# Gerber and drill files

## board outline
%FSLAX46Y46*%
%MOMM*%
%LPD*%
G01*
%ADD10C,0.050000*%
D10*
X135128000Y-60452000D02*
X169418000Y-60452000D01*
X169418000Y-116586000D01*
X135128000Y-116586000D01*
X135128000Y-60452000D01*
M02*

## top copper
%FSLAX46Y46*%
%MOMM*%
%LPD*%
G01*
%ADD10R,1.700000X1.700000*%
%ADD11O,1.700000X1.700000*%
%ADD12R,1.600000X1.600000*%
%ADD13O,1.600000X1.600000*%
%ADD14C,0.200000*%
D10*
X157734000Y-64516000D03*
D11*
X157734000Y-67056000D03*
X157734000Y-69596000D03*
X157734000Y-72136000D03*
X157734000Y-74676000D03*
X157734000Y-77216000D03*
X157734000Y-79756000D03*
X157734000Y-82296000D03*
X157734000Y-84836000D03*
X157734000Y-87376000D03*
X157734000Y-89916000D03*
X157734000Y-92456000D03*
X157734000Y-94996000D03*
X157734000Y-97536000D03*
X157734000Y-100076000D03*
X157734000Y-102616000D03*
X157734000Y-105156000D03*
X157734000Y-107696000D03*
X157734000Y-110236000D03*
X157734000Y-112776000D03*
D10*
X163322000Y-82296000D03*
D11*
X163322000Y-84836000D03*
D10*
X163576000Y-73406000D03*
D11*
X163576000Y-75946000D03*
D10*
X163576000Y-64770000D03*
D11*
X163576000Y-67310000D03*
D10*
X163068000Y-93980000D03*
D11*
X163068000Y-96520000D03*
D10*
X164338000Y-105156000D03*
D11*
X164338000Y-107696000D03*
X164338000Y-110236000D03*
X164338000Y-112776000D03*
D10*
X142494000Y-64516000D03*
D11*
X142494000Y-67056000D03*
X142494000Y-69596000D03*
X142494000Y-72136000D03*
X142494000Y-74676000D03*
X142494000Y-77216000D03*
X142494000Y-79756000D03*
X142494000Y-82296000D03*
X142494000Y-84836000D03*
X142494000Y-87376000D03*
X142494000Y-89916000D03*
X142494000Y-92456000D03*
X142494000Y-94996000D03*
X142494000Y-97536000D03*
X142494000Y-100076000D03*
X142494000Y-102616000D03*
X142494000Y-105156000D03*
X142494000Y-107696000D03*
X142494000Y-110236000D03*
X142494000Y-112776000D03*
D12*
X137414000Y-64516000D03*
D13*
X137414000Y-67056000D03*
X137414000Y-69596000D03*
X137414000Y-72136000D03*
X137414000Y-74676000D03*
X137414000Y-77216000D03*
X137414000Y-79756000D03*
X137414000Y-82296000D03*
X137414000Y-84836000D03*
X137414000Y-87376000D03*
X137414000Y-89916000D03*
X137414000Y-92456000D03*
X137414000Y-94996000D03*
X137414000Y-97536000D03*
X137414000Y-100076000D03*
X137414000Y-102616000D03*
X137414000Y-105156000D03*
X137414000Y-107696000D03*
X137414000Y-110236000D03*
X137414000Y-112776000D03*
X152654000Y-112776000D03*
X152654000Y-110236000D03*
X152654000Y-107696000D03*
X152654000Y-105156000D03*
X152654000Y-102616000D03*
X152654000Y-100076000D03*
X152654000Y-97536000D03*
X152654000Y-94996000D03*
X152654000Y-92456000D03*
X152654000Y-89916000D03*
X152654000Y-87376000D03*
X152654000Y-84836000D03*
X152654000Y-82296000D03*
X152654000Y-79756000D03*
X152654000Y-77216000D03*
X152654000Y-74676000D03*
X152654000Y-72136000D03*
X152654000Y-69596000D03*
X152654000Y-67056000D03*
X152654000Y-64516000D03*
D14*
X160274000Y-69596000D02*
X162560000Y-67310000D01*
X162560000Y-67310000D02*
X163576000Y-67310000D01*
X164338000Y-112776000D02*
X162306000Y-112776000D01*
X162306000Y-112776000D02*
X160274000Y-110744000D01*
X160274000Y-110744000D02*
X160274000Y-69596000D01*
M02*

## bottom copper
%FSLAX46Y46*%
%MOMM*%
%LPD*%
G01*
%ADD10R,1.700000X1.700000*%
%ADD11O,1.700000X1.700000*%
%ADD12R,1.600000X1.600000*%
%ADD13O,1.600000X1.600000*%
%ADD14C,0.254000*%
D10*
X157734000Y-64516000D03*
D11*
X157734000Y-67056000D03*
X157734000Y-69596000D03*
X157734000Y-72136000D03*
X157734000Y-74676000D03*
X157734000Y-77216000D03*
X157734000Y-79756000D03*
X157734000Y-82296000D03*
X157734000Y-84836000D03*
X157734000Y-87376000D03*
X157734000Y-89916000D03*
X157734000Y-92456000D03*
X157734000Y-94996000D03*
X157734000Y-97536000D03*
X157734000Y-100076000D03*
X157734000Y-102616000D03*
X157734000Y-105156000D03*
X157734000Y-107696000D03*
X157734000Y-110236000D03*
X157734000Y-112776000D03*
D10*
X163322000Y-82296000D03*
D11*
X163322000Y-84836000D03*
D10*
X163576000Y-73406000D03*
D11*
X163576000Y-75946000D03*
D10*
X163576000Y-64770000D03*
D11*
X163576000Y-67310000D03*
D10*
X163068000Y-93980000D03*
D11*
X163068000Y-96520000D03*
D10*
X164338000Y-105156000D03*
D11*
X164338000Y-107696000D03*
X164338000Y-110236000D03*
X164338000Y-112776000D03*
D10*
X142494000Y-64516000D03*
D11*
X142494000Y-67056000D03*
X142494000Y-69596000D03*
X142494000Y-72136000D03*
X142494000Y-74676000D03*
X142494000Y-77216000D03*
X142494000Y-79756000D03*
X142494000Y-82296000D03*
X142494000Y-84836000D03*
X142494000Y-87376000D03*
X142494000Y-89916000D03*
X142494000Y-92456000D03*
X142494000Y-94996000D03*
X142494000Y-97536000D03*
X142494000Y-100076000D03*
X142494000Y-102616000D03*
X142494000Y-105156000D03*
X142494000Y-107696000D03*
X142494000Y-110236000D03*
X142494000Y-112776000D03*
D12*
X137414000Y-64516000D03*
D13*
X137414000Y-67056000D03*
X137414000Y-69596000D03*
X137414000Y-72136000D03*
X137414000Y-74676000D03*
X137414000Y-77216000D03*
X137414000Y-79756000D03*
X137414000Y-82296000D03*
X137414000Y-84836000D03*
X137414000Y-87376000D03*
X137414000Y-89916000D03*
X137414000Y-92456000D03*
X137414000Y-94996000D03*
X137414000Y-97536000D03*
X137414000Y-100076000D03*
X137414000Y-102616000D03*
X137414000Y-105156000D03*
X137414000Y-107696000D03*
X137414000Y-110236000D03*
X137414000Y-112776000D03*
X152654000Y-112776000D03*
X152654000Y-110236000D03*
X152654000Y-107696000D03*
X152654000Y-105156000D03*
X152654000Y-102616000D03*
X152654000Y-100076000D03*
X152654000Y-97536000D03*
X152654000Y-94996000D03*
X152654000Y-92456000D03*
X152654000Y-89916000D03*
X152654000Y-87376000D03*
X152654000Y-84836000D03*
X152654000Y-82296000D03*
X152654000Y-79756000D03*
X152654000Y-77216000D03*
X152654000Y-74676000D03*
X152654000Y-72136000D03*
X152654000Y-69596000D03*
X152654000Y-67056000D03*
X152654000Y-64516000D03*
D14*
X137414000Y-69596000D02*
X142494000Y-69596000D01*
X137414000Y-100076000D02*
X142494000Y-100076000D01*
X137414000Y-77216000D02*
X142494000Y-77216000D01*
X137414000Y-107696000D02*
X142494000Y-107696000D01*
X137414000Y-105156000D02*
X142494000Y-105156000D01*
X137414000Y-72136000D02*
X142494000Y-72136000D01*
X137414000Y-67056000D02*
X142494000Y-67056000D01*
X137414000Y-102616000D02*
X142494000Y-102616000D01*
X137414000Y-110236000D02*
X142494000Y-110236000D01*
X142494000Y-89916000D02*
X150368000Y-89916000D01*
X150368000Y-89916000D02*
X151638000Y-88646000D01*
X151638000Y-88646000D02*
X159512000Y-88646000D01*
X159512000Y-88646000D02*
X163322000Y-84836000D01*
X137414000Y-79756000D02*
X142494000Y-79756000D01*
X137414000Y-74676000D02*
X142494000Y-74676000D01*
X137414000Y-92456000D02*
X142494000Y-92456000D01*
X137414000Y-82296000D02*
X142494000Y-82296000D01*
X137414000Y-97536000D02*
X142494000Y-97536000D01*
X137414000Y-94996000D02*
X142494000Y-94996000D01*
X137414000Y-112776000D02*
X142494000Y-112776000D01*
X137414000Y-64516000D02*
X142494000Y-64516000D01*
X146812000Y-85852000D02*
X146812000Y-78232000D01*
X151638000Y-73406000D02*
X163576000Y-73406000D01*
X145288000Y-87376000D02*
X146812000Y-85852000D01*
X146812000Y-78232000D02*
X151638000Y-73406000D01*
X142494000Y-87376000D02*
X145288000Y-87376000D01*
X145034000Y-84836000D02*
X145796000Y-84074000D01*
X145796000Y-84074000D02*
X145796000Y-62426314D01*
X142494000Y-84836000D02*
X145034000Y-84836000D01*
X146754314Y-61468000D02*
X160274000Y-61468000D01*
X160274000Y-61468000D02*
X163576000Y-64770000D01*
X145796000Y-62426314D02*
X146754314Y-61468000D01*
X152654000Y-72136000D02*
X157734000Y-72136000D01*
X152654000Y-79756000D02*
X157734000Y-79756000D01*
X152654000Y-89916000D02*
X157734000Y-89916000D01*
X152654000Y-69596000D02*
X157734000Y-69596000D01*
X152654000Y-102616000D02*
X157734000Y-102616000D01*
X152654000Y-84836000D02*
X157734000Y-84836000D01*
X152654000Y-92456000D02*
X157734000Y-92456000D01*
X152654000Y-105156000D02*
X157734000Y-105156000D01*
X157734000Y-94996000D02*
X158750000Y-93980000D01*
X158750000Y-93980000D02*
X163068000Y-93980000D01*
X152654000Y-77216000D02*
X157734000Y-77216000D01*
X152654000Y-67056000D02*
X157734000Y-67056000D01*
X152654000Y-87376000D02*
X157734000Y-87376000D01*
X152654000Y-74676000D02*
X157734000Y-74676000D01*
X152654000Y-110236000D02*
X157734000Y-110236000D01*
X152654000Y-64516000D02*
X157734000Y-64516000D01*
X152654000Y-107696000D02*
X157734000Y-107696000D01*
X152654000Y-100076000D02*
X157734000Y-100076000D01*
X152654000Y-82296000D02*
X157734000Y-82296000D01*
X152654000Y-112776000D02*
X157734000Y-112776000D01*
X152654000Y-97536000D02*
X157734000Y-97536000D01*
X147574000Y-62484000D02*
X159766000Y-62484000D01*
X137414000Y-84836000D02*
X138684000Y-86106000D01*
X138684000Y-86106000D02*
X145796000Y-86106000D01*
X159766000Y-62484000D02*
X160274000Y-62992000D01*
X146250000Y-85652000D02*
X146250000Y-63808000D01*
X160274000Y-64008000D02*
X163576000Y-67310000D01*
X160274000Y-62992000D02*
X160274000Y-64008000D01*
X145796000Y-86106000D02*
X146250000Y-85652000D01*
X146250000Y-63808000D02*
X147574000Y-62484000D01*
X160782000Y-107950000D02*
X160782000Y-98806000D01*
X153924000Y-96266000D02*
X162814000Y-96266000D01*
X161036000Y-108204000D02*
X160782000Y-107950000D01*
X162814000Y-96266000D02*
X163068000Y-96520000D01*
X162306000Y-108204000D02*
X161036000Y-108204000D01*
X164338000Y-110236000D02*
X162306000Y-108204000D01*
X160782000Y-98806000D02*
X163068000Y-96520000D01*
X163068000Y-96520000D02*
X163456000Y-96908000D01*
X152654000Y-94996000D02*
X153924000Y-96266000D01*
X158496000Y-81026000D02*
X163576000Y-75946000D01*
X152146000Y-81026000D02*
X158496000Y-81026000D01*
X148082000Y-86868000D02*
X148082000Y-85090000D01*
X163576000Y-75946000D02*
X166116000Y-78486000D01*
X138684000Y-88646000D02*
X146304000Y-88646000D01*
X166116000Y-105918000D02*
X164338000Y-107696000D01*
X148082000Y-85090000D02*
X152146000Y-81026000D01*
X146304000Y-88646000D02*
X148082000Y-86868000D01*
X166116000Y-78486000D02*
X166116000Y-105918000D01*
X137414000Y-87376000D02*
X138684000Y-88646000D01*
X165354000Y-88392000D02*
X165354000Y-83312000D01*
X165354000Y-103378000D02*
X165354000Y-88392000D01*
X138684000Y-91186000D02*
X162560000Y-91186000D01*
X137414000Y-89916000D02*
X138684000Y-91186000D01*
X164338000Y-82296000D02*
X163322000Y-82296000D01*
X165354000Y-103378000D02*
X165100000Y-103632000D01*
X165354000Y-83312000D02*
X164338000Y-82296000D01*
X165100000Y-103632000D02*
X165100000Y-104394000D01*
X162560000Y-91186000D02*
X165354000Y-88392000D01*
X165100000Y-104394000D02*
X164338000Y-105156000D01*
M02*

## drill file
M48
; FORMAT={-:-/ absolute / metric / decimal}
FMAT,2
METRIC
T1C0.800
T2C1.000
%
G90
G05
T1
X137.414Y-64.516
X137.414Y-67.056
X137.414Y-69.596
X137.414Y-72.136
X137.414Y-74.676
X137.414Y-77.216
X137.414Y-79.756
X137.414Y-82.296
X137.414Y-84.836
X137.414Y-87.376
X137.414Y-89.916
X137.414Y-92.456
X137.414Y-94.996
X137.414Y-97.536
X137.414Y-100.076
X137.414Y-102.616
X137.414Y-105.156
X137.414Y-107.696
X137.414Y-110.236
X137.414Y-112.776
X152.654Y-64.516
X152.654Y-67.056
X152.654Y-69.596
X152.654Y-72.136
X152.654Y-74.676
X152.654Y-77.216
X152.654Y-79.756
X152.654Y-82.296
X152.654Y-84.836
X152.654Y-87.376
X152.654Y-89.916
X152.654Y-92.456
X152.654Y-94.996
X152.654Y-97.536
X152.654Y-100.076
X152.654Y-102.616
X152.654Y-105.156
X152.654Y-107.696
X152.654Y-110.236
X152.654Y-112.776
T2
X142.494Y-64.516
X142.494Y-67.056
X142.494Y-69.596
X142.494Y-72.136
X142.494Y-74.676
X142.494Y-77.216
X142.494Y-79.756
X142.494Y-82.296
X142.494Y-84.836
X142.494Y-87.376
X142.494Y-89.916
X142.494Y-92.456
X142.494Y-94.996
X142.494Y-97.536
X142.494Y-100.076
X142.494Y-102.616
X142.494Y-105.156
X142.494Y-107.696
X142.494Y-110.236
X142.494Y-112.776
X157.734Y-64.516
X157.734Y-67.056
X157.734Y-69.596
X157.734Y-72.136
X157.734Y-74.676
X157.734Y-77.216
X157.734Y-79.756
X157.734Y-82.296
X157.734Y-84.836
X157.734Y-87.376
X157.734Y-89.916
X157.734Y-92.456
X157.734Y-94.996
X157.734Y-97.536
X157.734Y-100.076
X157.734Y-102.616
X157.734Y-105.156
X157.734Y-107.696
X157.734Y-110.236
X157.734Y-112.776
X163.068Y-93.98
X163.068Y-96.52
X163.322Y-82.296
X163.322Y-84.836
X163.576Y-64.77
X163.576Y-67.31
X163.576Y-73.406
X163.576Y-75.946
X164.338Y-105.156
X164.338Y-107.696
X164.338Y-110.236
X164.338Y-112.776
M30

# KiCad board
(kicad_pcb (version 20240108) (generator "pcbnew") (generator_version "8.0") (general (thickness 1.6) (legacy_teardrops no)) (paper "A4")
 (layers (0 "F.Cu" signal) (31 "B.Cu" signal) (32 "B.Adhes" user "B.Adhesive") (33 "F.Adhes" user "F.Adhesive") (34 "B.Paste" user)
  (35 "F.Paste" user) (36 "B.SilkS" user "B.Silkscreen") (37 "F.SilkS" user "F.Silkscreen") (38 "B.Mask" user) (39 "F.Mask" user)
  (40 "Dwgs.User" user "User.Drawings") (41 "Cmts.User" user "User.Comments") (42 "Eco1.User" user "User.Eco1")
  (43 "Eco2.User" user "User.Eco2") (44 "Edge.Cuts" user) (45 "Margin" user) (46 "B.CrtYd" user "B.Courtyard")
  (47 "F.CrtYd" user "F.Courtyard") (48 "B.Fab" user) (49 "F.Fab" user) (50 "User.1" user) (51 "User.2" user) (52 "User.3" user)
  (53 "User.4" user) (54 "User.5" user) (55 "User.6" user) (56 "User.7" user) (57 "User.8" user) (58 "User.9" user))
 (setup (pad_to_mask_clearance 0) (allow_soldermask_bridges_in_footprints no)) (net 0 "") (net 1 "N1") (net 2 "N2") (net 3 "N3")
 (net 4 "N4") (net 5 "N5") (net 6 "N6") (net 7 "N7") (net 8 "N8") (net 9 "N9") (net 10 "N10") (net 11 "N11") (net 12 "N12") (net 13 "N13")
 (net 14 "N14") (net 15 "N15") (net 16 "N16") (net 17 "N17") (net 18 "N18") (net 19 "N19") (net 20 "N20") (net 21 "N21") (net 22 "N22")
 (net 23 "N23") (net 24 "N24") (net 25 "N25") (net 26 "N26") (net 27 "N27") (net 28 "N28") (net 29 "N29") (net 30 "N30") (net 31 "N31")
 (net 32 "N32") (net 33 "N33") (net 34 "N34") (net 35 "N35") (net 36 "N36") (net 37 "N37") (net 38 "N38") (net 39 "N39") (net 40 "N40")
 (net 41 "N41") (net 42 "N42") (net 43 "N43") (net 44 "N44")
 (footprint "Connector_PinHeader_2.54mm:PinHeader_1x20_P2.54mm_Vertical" (layer "F.Cu") (at 157.734 64.516)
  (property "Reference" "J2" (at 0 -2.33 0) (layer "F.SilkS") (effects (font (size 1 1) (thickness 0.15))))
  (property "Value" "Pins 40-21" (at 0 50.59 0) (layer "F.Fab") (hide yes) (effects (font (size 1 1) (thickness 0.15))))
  (pad "1" thru_hole rect (at 0 0) (size 1.7 1.7) (drill 1) (layers "*.Cu" "*.Mask") (remove_unused_layers no) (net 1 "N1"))
  (pad "2" thru_hole oval (at 0 2.54) (size 1.7 1.7) (drill 1) (layers "*.Cu" "*.Mask") (remove_unused_layers no) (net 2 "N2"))
  (pad "3" thru_hole oval (at 0 5.08) (size 1.7 1.7) (drill 1) (layers "*.Cu" "*.Mask") (remove_unused_layers no) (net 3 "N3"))
  (pad "4" thru_hole oval (at 0 7.62) (size 1.7 1.7) (drill 1) (layers "*.Cu" "*.Mask") (remove_unused_layers no) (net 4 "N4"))
  (pad "5" thru_hole oval (at 0 10.16) (size 1.7 1.7) (drill 1) (layers "*.Cu" "*.Mask") (remove_unused_layers no) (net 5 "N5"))
  (pad "6" thru_hole oval (at 0 12.7) (size 1.7 1.7) (drill 1) (layers "*.Cu" "*.Mask") (remove_unused_layers no) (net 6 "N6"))
  (pad "7" thru_hole oval (at 0 15.24) (size 1.7 1.7) (drill 1) (layers "*.Cu" "*.Mask") (remove_unused_layers no) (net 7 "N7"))
  (pad "8" thru_hole oval (at 0 17.78) (size 1.7 1.7) (drill 1) (layers "*.Cu" "*.Mask") (remove_unused_layers no) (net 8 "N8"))
  (pad "9" thru_hole oval (at 0 20.32) (size 1.7 1.7) (drill 1) (layers "*.Cu" "*.Mask") (remove_unused_layers no) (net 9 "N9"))
  (pad "10" thru_hole oval (at 0 22.86) (size 1.7 1.7) (drill 1) (layers "*.Cu" "*.Mask") (remove_unused_layers no) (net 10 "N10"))
  (pad "11" thru_hole oval (at 0 25.4) (size 1.7 1.7) (drill 1) (layers "*.Cu" "*.Mask") (remove_unused_layers no) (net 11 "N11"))
  (pad "12" thru_hole oval (at 0 27.94) (size 1.7 1.7) (drill 1) (layers "*.Cu" "*.Mask") (remove_unused_layers no) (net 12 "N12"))
  (pad "13" thru_hole oval (at 0 30.48) (size 1.7 1.7) (drill 1) (layers "*.Cu" "*.Mask") (remove_unused_layers no) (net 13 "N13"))
  (pad "14" thru_hole oval (at 0 33.02) (size 1.7 1.7) (drill 1) (layers "*.Cu" "*.Mask") (remove_unused_layers no) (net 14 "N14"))
  (pad "15" thru_hole oval (at 0 35.56) (size 1.7 1.7) (drill 1) (layers "*.Cu" "*.Mask") (remove_unused_layers no) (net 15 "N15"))
  (pad "16" thru_hole oval (at 0 38.1) (size 1.7 1.7) (drill 1) (layers "*.Cu" "*.Mask") (remove_unused_layers no) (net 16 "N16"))
  (pad "17" thru_hole oval (at 0 40.64) (size 1.7 1.7) (drill 1) (layers "*.Cu" "*.Mask") (remove_unused_layers no) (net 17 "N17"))
  (pad "18" thru_hole oval (at 0 43.18) (size 1.7 1.7) (drill 1) (layers "*.Cu" "*.Mask") (remove_unused_layers no) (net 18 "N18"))
  (pad "19" thru_hole oval (at 0 45.72) (size 1.7 1.7) (drill 1) (layers "*.Cu" "*.Mask") (remove_unused_layers no) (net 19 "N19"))
  (pad "20" thru_hole oval (at 0 48.26) (size 1.7 1.7) (drill 1) (layers "*.Cu" "*.Mask") (remove_unused_layers no) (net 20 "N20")))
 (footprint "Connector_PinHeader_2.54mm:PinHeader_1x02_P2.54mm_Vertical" (layer "F.Cu") (at 163.322 82.296)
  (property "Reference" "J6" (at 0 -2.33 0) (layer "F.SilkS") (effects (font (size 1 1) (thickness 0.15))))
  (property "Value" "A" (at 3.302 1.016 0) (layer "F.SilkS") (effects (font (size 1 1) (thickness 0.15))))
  (pad "1" thru_hole rect (at 0 0) (size 1.7 1.7) (drill 1) (layers "*.Cu" "*.Mask") (remove_unused_layers no) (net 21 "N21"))
  (pad "2" thru_hole oval (at 0 2.54) (size 1.7 1.7) (drill 1) (layers "*.Cu" "*.Mask") (remove_unused_layers no) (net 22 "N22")))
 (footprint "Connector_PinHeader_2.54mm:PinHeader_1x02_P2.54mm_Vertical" (layer "F.Cu") (at 163.576 73.406)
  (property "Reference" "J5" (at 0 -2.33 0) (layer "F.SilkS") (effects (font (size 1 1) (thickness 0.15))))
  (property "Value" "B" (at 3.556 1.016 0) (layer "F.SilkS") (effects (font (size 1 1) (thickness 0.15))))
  (pad "1" thru_hole rect (at 0 0) (size 1.7 1.7) (drill 1) (layers "*.Cu" "*.Mask") (remove_unused_layers no) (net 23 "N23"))
  (pad "2" thru_hole oval (at 0 2.54) (size 1.7 1.7) (drill 1) (layers "*.Cu" "*.Mask") (remove_unused_layers no) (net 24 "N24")))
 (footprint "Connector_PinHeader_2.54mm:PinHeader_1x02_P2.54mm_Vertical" (layer "F.Cu") (at 163.576 64.77)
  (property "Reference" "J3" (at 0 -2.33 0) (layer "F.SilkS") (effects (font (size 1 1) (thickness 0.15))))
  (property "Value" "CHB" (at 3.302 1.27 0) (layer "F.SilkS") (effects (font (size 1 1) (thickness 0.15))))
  (pad "1" thru_hole rect (at 0 0) (size 1.7 1.7) (drill 1) (layers "*.Cu" "*.Mask") (remove_unused_layers no) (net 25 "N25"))
  (pad "2" thru_hole oval (at 0 2.54) (size 1.7 1.7) (drill 1) (layers "*.Cu" "*.Mask") (remove_unused_layers no) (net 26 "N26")))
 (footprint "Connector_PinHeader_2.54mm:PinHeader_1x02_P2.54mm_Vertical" (layer "F.Cu") (at 163.068 93.98)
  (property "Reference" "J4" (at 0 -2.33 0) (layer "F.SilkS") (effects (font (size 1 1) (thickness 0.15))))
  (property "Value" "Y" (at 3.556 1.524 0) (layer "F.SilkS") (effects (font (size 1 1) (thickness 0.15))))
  (pad "1" thru_hole rect (at 0 0) (size 1.7 1.7) (drill 1) (layers "*.Cu" "*.Mask") (remove_unused_layers no) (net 13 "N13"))
  (pad "2" thru_hole oval (at 0 2.54) (size 1.7 1.7) (drill 1) (layers "*.Cu" "*.Mask") (remove_unused_layers no) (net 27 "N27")))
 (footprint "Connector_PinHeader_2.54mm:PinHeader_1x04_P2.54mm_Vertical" (layer "F.Cu") (at 164.338 105.156)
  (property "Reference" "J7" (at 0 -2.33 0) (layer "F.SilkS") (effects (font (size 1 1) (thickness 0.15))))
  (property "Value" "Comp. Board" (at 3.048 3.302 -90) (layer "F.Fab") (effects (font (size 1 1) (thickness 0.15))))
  (pad "1" thru_hole rect (at 0 0) (size 1.7 1.7) (drill 1) (layers "*.Cu" "*.Mask") (remove_unused_layers no) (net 21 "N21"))
  (pad "2" thru_hole oval (at 0 2.54) (size 1.7 1.7) (drill 1) (layers "*.Cu" "*.Mask") (remove_unused_layers no) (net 24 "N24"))
  (pad "3" thru_hole oval (at 0 5.08) (size 1.7 1.7) (drill 1) (layers "*.Cu" "*.Mask") (remove_unused_layers no) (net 27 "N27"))
  (pad "4" thru_hole oval (at 0 7.62) (size 1.7 1.7) (drill 1) (layers "*.Cu" "*.Mask") (remove_unused_layers no) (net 26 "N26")))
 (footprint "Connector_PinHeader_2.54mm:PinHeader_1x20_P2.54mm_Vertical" (layer "F.Cu") (at 142.494 64.516)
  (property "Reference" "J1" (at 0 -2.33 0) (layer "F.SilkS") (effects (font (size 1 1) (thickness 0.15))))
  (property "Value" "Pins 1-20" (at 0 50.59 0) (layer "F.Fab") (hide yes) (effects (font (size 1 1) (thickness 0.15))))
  (pad "1" thru_hole rect (at 0 0) (size 1.7 1.7) (drill 1) (layers "*.Cu" "*.Mask") (remove_unused_layers no) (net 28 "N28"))
  (pad "2" thru_hole oval (at 0 2.54) (size 1.7 1.7) (drill 1) (layers "*.Cu" "*.Mask") (remove_unused_layers no) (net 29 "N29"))
  (pad "3" thru_hole oval (at 0 5.08) (size 1.7 1.7) (drill 1) (layers "*.Cu" "*.Mask") (remove_unused_layers no) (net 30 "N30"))
  (pad "4" thru_hole oval (at 0 7.62) (size 1.7 1.7) (drill 1) (layers "*.Cu" "*.Mask") (remove_unused_layers no) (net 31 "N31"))
  (pad "5" thru_hole oval (at 0 10.16) (size 1.7 1.7) (drill 1) (layers "*.Cu" "*.Mask") (remove_unused_layers no) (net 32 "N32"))
  (pad "6" thru_hole oval (at 0 12.7) (size 1.7 1.7) (drill 1) (layers "*.Cu" "*.Mask") (remove_unused_layers no) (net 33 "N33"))
  (pad "7" thru_hole oval (at 0 15.24) (size 1.7 1.7) (drill 1) (layers "*.Cu" "*.Mask") (remove_unused_layers no) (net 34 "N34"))
  (pad "8" thru_hole oval (at 0 17.78) (size 1.7 1.7) (drill 1) (layers "*.Cu" "*.Mask") (remove_unused_layers no) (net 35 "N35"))
  (pad "9" thru_hole oval (at 0 20.32) (size 1.7 1.7) (drill 1) (layers "*.Cu" "*.Mask") (remove_unused_layers no) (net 25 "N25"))
  (pad "10" thru_hole oval (at 0 22.86) (size 1.7 1.7) (drill 1) (layers "*.Cu" "*.Mask") (remove_unused_layers no) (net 23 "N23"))
  (pad "11" thru_hole oval (at 0 25.4) (size 1.7 1.7) (drill 1) (layers "*.Cu" "*.Mask") (remove_unused_layers no) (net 22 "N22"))
  (pad "12" thru_hole oval (at 0 27.94) (size 1.7 1.7) (drill 1) (layers "*.Cu" "*.Mask") (remove_unused_layers no) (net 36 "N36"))
  (pad "13" thru_hole oval (at 0 30.48) (size 1.7 1.7) (drill 1) (layers "*.Cu" "*.Mask") (remove_unused_layers no) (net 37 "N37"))
  (pad "14" thru_hole oval (at 0 33.02) (size 1.7 1.7) (drill 1) (layers "*.Cu" "*.Mask") (remove_unused_layers no) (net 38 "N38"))
  (pad "15" thru_hole oval (at 0 35.56) (size 1.7 1.7) (drill 1) (layers "*.Cu" "*.Mask") (remove_unused_layers no) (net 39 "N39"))
  (pad "16" thru_hole oval (at 0 38.1) (size 1.7 1.7) (drill 1) (layers "*.Cu" "*.Mask") (remove_unused_layers no) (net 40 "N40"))
  (pad "17" thru_hole oval (at 0 40.64) (size 1.7 1.7) (drill 1) (layers "*.Cu" "*.Mask") (remove_unused_layers no) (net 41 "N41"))
  (pad "18" thru_hole oval (at 0 43.18) (size 1.7 1.7) (drill 1) (layers "*.Cu" "*.Mask") (remove_unused_layers no) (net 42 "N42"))
  (pad "19" thru_hole oval (at 0 45.72) (size 1.7 1.7) (drill 1) (layers "*.Cu" "*.Mask") (remove_unused_layers no) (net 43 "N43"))
  (pad "20" thru_hole oval (at 0 48.26) (size 1.7 1.7) (drill 1) (layers "*.Cu" "*.Mask") (remove_unused_layers no) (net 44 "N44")))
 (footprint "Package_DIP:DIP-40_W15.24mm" (layer "F.Cu") (at 137.414 64.516)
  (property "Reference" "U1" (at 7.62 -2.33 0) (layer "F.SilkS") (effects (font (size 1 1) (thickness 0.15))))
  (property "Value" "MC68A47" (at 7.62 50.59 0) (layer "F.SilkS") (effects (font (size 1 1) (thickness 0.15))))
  (pad "1" thru_hole rect (at 0 0) (size 1.6 1.6) (drill 0.8) (layers "*.Cu" "*.Mask") (remove_unused_layers no) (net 28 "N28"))
  (pad "2" thru_hole oval (at 0 2.54) (size 1.6 1.6) (drill 0.8) (layers "*.Cu" "*.Mask") (remove_unused_layers no) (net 29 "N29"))
  (pad "3" thru_hole oval (at 0 5.08) (size 1.6 1.6) (drill 0.8) (layers "*.Cu" "*.Mask") (remove_unused_layers no) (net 30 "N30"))
  (pad "4" thru_hole oval (at 0 7.62) (size 1.6 1.6) (drill 0.8) (layers "*.Cu" "*.Mask") (remove_unused_layers no) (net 31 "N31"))
  (pad "5" thru_hole oval (at 0 10.16) (size 1.6 1.6) (drill 0.8) (layers "*.Cu" "*.Mask") (remove_unused_layers no) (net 32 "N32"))
  (pad "6" thru_hole oval (at 0 12.7) (size 1.6 1.6) (drill 0.8) (layers "*.Cu" "*.Mask") (remove_unused_layers no) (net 33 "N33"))
  (pad "7" thru_hole oval (at 0 15.24) (size 1.6 1.6) (drill 0.8) (layers "*.Cu" "*.Mask") (remove_unused_layers no) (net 34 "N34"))
  (pad "8" thru_hole oval (at 0 17.78) (size 1.6 1.6) (drill 0.8) (layers "*.Cu" "*.Mask") (remove_unused_layers no) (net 35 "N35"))
  (pad "9" thru_hole oval (at 0 20.32) (size 1.6 1.6) (drill 0.8) (layers "*.Cu" "*.Mask") (remove_unused_layers no) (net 26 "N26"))
  (pad "10" thru_hole oval (at 0 22.86) (size 1.6 1.6) (drill 0.8) (layers "*.Cu" "*.Mask") (remove_unused_layers no) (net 24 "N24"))
  (pad "11" thru_hole oval (at 0 25.4) (size 1.6 1.6) (drill 0.8) (layers "*.Cu" "*.Mask") (remove_unused_layers no) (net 21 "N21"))
  (pad "12" thru_hole oval (at 0 27.94) (size 1.6 1.6) (drill 0.8) (layers "*.Cu" "*.Mask") (remove_unused_layers no) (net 36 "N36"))
  (pad "13" thru_hole oval (at 0 30.48) (size 1.6 1.6) (drill 0.8) (layers "*.Cu" "*.Mask") (remove_unused_layers no) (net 37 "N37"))
  (pad "14" thru_hole oval (at 0 33.02) (size 1.6 1.6) (drill 0.8) (layers "*.Cu" "*.Mask") (remove_unused_layers no) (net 38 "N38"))
  (pad "15" thru_hole oval (at 0 35.56) (size 1.6 1.6) (drill 0.8) (layers "*.Cu" "*.Mask") (remove_unused_layers no) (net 39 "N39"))
  (pad "16" thru_hole oval (at 0 38.1) (size 1.6 1.6) (drill 0.8) (layers "*.Cu" "*.Mask") (remove_unused_layers no) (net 40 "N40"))
  (pad "17" thru_hole oval (at 0 40.64) (size 1.6 1.6) (drill 0.8) (layers "*.Cu" "*.Mask") (remove_unused_layers no) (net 41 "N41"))
  (pad "18" thru_hole oval (at 0 43.18) (size 1.6 1.6) (drill 0.8) (layers "*.Cu" "*.Mask") (remove_unused_layers no) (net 42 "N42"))
  (pad "19" thru_hole oval (at 0 45.72) (size 1.6 1.6) (drill 0.8) (layers "*.Cu" "*.Mask") (remove_unused_layers no) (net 43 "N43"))
  (pad "20" thru_hole oval (at 0 48.26) (size 1.6 1.6) (drill 0.8) (layers "*.Cu" "*.Mask") (remove_unused_layers no) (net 44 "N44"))
  (pad "21" thru_hole oval (at 15.24 48.26) (size 1.6 1.6) (drill 0.8) (layers "*.Cu" "*.Mask") (remove_unused_layers no) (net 20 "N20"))
  (pad "22" thru_hole oval (at 15.24 45.72) (size 1.6 1.6) (drill 0.8) (layers "*.Cu" "*.Mask") (remove_unused_layers no) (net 19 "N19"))
  (pad "23" thru_hole oval (at 15.24 43.18) (size 1.6 1.6) (drill 0.8) (layers "*.Cu" "*.Mask") (remove_unused_layers no) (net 18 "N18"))
  (pad "24" thru_hole oval (at 15.24 40.64) (size 1.6 1.6) (drill 0.8) (layers "*.Cu" "*.Mask") (remove_unused_layers no) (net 17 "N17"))
  (pad "25" thru_hole oval (at 15.24 38.1) (size 1.6 1.6) (drill 0.8) (layers "*.Cu" "*.Mask") (remove_unused_layers no) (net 16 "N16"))
  (pad "26" thru_hole oval (at 15.24 35.56) (size 1.6 1.6) (drill 0.8) (layers "*.Cu" "*.Mask") (remove_unused_layers no) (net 15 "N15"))
  (pad "27" thru_hole oval (at 15.24 33.02) (size 1.6 1.6) (drill 0.8) (layers "*.Cu" "*.Mask") (remove_unused_layers no) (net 14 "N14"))
  (pad "28" thru_hole oval (at 15.24 30.48) (size 1.6 1.6) (drill 0.8) (layers "*.Cu" "*.Mask") (remove_unused_layers no) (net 27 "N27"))
  (pad "29" thru_hole oval (at 15.24 27.94) (size 1.6 1.6) (drill 0.8) (layers "*.Cu" "*.Mask") (remove_unused_layers no) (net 12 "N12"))
  (pad "30" thru_hole oval (at 15.24 25.4) (size 1.6 1.6) (drill 0.8) (layers "*.Cu" "*.Mask") (remove_unused_layers no) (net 11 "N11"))
  (pad "31" thru_hole oval (at 15.24 22.86) (size 1.6 1.6) (drill 0.8) (layers "*.Cu" "*.Mask") (remove_unused_layers no) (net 10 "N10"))
  (pad "32" thru_hole oval (at 15.24 20.32) (size 1.6 1.6) (drill 0.8) (layers "*.Cu" "*.Mask") (remove_unused_layers no) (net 9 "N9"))
  (pad "33" thru_hole oval (at 15.24 17.78) (size 1.6 1.6) (drill 0.8) (layers "*.Cu" "*.Mask") (remove_unused_layers no) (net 8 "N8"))
  (pad "34" thru_hole oval (at 15.24 15.24) (size 1.6 1.6) (drill 0.8) (layers "*.Cu" "*.Mask") (remove_unused_layers no) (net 7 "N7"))
  (pad "35" thru_hole oval (at 15.24 12.7) (size 1.6 1.6) (drill 0.8) (layers "*.Cu" "*.Mask") (remove_unused_layers no) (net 6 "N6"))
  (pad "36" thru_hole oval (at 15.24 10.16) (size 1.6 1.6) (drill 0.8) (layers "*.Cu" "*.Mask") (remove_unused_layers no) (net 5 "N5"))
  (pad "37" thru_hole oval (at 15.24 7.62) (size 1.6 1.6) (drill 0.8) (layers "*.Cu" "*.Mask") (remove_unused_layers no) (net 4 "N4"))
  (pad "38" thru_hole oval (at 15.24 5.08) (size 1.6 1.6) (drill 0.8) (layers "*.Cu" "*.Mask") (remove_unused_layers no) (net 3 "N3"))
  (pad "39" thru_hole oval (at 15.24 2.54) (size 1.6 1.6) (drill 0.8) (layers "*.Cu" "*.Mask") (remove_unused_layers no) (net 2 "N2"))
  (pad "40" thru_hole oval (at 15.24 0) (size 1.6 1.6) (drill 0.8) (layers "*.Cu" "*.Mask") (remove_unused_layers no) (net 1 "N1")))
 (gr_rect (start 135.128 60.452) (end 169.418 116.586) (stroke (width 0.05) (type default)) (fill none) (layer "Edge.Cuts"))
 (segment (start 137.414 69.596) (end 142.494 69.596) (width 0.254) (layer "B.Cu") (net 30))
 (segment (start 137.414 100.076) (end 142.494 100.076) (width 0.254) (layer "B.Cu") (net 39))
 (segment (start 137.414 77.216) (end 142.494 77.216) (width 0.254) (layer "B.Cu") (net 33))
 (segment (start 137.414 107.696) (end 142.494 107.696) (width 0.254) (layer "B.Cu") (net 42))
 (segment (start 137.414 105.156) (end 142.494 105.156) (width 0.254) (layer "B.Cu") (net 41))
 (segment (start 137.414 72.136) (end 142.494 72.136) (width 0.254) (layer "B.Cu") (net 31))
 (segment (start 137.414 67.056) (end 142.494 67.056) (width 0.254) (layer "B.Cu") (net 29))
 (segment (start 137.414 102.616) (end 142.494 102.616) (width 0.254) (layer "B.Cu") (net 40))
 (segment (start 137.414 110.236) (end 142.494 110.236) (width 0.254) (layer "B.Cu") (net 43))
 (segment (start 142.494 89.916) (end 150.368 89.916) (width 0.254) (layer "B.Cu") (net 22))
 (segment (start 150.368 89.916) (end 151.638 88.646) (width 0.254) (layer "B.Cu") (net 22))
 (segment (start 151.638 88.646) (end 159.512 88.646) (width 0.254) (layer "B.Cu") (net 22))
 (segment (start 159.512 88.646) (end 163.322 84.836) (width 0.254) (layer "B.Cu") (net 22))
 (segment (start 137.414 79.756) (end 142.494 79.756) (width 0.254) (layer "B.Cu") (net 34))
 (segment (start 137.414 74.676) (end 142.494 74.676) (width 0.254) (layer "B.Cu") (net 32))
 (segment (start 137.414 92.456) (end 142.494 92.456) (width 0.254) (layer "B.Cu") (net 36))
 (segment (start 137.414 82.296) (end 142.494 82.296) (width 0.254) (layer "B.Cu") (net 35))
 (segment (start 137.414 97.536) (end 142.494 97.536) (width 0.254) (layer "B.Cu") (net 38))
 (segment (start 137.414 94.996) (end 142.494 94.996) (width 0.254) (layer "B.Cu") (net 37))
 (segment (start 137.414 112.776) (end 142.494 112.776) (width 0.254) (layer "B.Cu") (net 44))
 (segment (start 137.414 64.516) (end 142.494 64.516) (width 0.254) (layer "B.Cu") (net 28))
 (segment (start 146.812 85.852) (end 146.812 78.232) (width 0.254) (layer "B.Cu") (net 23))
 (segment (start 151.638 73.406) (end 163.576 73.406) (width 0.254) (layer "B.Cu") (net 23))
 (segment (start 145.288 87.376) (end 146.812 85.852) (width 0.254) (layer "B.Cu") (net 23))
 (segment (start 146.812 78.232) (end 151.638 73.406) (width 0.254) (layer "B.Cu") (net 23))
 (segment (start 142.494 87.376) (end 145.288 87.376) (width 0.254) (layer "B.Cu") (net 23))
 (segment (start 145.034 84.836) (end 145.796 84.074) (width 0.254) (layer "B.Cu") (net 25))
 (segment (start 145.796 84.074) (end 145.796 62.426314) (width 0.254) (layer "B.Cu") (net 25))
 (segment (start 142.494 84.836) (end 145.034 84.836) (width 0.254) (layer "B.Cu") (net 25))
 (segment (start 146.754314 61.468) (end 160.274 61.468) (width 0.254) (layer "B.Cu") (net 25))
 (segment (start 160.274 61.468) (end 163.576 64.77) (width 0.254) (layer "B.Cu") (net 25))
 (segment (start 145.796 62.426314) (end 146.754314 61.468) (width 0.254) (layer "B.Cu") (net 25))
 (segment (start 152.654 72.136) (end 157.734 72.136) (width 0.254) (layer "B.Cu") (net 4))
 (segment (start 152.654 79.756) (end 157.734 79.756) (width 0.254) (layer "B.Cu") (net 7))
 (segment (start 152.654 89.916) (end 157.734 89.916) (width 0.254) (layer "B.Cu") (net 11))
 (segment (start 152.654 69.596) (end 157.734 69.596) (width 0.254) (layer "B.Cu") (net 3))
 (segment (start 152.654 102.616) (end 157.734 102.616) (width 0.254) (layer "B.Cu") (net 16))
 (segment (start 152.654 84.836) (end 157.734 84.836) (width 0.254) (layer "B.Cu") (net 9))
 (segment (start 152.654 92.456) (end 157.734 92.456) (width 0.254) (layer "B.Cu") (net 12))
 (segment (start 152.654 105.156) (end 157.734 105.156) (width 0.254) (layer "B.Cu") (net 17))
 (segment (start 157.734 94.996) (end 158.75 93.98) (width 0.254) (layer "B.Cu") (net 13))
 (segment (start 158.75 93.98) (end 163.068 93.98) (width 0.254) (layer "B.Cu") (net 13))
 (segment (start 152.654 77.216) (end 157.734 77.216) (width 0.254) (layer "B.Cu") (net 6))
 (segment (start 152.654 67.056) (end 157.734 67.056) (width 0.254) (layer "B.Cu") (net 2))
 (segment (start 152.654 87.376) (end 157.734 87.376) (width 0.254) (layer "B.Cu") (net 10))
 (segment (start 152.654 74.676) (end 157.734 74.676) (width 0.254) (layer "B.Cu") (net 5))
 (segment (start 152.654 110.236) (end 157.734 110.236) (width 0.254) (layer "B.Cu") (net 19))
 (segment (start 152.654 64.516) (end 157.734 64.516) (width 0.254) (layer "B.Cu") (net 1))
 (segment (start 152.654 107.696) (end 157.734 107.696) (width 0.254) (layer "B.Cu") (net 18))
 (segment (start 152.654 100.076) (end 157.734 100.076) (width 0.254) (layer "B.Cu") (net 15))
 (segment (start 152.654 82.296) (end 157.734 82.296) (width 0.254) (layer "B.Cu") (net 8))
 (segment (start 152.654 112.776) (end 157.734 112.776) (width 0.254) (layer "B.Cu") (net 20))
 (segment (start 152.654 97.536) (end 157.734 97.536) (width 0.254) (layer "B.Cu") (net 14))
 (segment (start 160.274 69.596) (end 162.56 67.31) (width 0.2) (layer "F.Cu") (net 26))
 (segment (start 162.56 67.31) (end 163.576 67.31) (width 0.2) (layer "F.Cu") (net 26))
 (segment (start 164.338 112.776) (end 162.306 112.776) (width 0.2) (layer "F.Cu") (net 26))
 (segment (start 162.306 112.776) (end 160.274 110.744) (width 0.2) (layer "F.Cu") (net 26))
 (segment (start 160.274 110.744) (end 160.274 69.596) (width 0.2) (layer "F.Cu") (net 26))
 (segment (start 147.574 62.484) (end 159.766 62.484) (width 0.254) (layer "B.Cu") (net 26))
 (segment (start 137.414 84.836) (end 138.684 86.106) (width 0.254) (layer "B.Cu") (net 26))
 (segment (start 138.684 86.106) (end 145.796 86.106) (width 0.254) (layer "B.Cu") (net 26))
 (segment (start 159.766 62.484) (end 160.274 62.992) (width 0.254) (layer "B.Cu") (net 26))
 (segment (start 146.25 85.652) (end 146.25 63.808) (width 0.254) (layer "B.Cu") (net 26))
 (segment (start 160.274 64.008) (end 163.576 67.31) (width 0.254) (layer "B.Cu") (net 26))
 (segment (start 160.274 62.992) (end 160.274 64.008) (width 0.254) (layer "B.Cu") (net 26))
 (segment (start 145.796 86.106) (end 146.25 85.652) (width 0.254) (layer "B.Cu") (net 26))
 (segment (start 146.25 63.808) (end 147.574 62.484) (width 0.254) (layer "B.Cu") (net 26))
 (segment (start 160.782 107.95) (end 160.782 98.806) (width 0.254) (layer "B.Cu") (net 27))
 (segment (start 153.924 96.266) (end 162.814 96.266) (width 0.254) (layer "B.Cu") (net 27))
 (segment (start 161.036 108.204) (end 160.782 107.95) (width 0.254) (layer "B.Cu") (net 27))
 (segment (start 162.814 96.266) (end 163.068 96.52) (width 0.254) (layer "B.Cu") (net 27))
 (segment (start 162.306 108.204) (end 161.036 108.204) (width 0.254) (layer "B.Cu") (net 27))
 (segment (start 164.338 110.236) (end 162.306 108.204) (width 0.254) (layer "B.Cu") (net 27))
 (segment (start 160.782 98.806) (end 163.068 96.52) (width 0.254) (layer "B.Cu") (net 27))
 (segment (start 163.068 96.52) (end 163.456 96.908) (width 0.254) (layer "B.Cu") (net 27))
 (segment (start 152.654 94.996) (end 153.924 96.266) (width 0.254) (layer "B.Cu") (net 27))
 (segment (start 158.496 81.026) (end 163.576 75.946) (width 0.254) (layer "B.Cu") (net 24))
 (segment (start 152.146 81.026) (end 158.496 81.026) (width 0.254) (layer "B.Cu") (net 24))
 (segment (start 148.082 86.868) (end 148.082 85.09) (width 0.254) (layer "B.Cu") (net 24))
 (segment (start 163.576 75.946) (end 166.116 78.486) (width 0.254) (layer "B.Cu") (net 24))
 (segment (start 138.684 88.646) (end 146.304 88.646) (width 0.254) (layer "B.Cu") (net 24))
 (segment (start 166.116 105.918) (end 164.338 107.696) (width 0.254) (layer "B.Cu") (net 24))
 (segment (start 148.082 85.09) (end 152.146 81.026) (width 0.254) (layer "B.Cu") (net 24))
 (segment (start 146.304 88.646) (end 148.082 86.868) (width 0.254) (layer "B.Cu") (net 24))
 (segment (start 166.116 78.486) (end 166.116 105.918) (width 0.254) (layer "B.Cu") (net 24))
 (segment (start 137.414 87.376) (end 138.684 88.646) (width 0.254) (layer "B.Cu") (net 24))
 (segment (start 165.354 88.392) (end 165.354 83.312) (width 0.254) (layer "B.Cu") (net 21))
 (segment (start 165.354 103.378) (end 165.354 88.392) (width 0.254) (layer "B.Cu") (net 21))
 (segment (start 138.684 91.186) (end 162.56 91.186) (width 0.254) (layer "B.Cu") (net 21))
 (segment (start 137.414 89.916) (end 138.684 91.186) (width 0.254) (layer "B.Cu") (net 21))
 (segment (start 164.338 82.296) (end 163.322 82.296) (width 0.254) (layer "B.Cu") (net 21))
 (segment (start 165.354 103.378) (end 165.1 103.632) (width 0.254) (layer "B.Cu") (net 21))
 (segment (start 165.354 83.312) (end 164.338 82.296) (width 0.254) (layer "B.Cu") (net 21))
 (segment (start 165.1 103.632) (end 165.1 104.394) (width 0.254) (layer "B.Cu") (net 21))
 (segment (start 162.56 91.186) (end 165.354 88.392) (width 0.254) (layer "B.Cu") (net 21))
 (segment (start 165.1 104.394) (end 164.338 105.156) (width 0.254) (layer "B.Cu") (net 21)))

